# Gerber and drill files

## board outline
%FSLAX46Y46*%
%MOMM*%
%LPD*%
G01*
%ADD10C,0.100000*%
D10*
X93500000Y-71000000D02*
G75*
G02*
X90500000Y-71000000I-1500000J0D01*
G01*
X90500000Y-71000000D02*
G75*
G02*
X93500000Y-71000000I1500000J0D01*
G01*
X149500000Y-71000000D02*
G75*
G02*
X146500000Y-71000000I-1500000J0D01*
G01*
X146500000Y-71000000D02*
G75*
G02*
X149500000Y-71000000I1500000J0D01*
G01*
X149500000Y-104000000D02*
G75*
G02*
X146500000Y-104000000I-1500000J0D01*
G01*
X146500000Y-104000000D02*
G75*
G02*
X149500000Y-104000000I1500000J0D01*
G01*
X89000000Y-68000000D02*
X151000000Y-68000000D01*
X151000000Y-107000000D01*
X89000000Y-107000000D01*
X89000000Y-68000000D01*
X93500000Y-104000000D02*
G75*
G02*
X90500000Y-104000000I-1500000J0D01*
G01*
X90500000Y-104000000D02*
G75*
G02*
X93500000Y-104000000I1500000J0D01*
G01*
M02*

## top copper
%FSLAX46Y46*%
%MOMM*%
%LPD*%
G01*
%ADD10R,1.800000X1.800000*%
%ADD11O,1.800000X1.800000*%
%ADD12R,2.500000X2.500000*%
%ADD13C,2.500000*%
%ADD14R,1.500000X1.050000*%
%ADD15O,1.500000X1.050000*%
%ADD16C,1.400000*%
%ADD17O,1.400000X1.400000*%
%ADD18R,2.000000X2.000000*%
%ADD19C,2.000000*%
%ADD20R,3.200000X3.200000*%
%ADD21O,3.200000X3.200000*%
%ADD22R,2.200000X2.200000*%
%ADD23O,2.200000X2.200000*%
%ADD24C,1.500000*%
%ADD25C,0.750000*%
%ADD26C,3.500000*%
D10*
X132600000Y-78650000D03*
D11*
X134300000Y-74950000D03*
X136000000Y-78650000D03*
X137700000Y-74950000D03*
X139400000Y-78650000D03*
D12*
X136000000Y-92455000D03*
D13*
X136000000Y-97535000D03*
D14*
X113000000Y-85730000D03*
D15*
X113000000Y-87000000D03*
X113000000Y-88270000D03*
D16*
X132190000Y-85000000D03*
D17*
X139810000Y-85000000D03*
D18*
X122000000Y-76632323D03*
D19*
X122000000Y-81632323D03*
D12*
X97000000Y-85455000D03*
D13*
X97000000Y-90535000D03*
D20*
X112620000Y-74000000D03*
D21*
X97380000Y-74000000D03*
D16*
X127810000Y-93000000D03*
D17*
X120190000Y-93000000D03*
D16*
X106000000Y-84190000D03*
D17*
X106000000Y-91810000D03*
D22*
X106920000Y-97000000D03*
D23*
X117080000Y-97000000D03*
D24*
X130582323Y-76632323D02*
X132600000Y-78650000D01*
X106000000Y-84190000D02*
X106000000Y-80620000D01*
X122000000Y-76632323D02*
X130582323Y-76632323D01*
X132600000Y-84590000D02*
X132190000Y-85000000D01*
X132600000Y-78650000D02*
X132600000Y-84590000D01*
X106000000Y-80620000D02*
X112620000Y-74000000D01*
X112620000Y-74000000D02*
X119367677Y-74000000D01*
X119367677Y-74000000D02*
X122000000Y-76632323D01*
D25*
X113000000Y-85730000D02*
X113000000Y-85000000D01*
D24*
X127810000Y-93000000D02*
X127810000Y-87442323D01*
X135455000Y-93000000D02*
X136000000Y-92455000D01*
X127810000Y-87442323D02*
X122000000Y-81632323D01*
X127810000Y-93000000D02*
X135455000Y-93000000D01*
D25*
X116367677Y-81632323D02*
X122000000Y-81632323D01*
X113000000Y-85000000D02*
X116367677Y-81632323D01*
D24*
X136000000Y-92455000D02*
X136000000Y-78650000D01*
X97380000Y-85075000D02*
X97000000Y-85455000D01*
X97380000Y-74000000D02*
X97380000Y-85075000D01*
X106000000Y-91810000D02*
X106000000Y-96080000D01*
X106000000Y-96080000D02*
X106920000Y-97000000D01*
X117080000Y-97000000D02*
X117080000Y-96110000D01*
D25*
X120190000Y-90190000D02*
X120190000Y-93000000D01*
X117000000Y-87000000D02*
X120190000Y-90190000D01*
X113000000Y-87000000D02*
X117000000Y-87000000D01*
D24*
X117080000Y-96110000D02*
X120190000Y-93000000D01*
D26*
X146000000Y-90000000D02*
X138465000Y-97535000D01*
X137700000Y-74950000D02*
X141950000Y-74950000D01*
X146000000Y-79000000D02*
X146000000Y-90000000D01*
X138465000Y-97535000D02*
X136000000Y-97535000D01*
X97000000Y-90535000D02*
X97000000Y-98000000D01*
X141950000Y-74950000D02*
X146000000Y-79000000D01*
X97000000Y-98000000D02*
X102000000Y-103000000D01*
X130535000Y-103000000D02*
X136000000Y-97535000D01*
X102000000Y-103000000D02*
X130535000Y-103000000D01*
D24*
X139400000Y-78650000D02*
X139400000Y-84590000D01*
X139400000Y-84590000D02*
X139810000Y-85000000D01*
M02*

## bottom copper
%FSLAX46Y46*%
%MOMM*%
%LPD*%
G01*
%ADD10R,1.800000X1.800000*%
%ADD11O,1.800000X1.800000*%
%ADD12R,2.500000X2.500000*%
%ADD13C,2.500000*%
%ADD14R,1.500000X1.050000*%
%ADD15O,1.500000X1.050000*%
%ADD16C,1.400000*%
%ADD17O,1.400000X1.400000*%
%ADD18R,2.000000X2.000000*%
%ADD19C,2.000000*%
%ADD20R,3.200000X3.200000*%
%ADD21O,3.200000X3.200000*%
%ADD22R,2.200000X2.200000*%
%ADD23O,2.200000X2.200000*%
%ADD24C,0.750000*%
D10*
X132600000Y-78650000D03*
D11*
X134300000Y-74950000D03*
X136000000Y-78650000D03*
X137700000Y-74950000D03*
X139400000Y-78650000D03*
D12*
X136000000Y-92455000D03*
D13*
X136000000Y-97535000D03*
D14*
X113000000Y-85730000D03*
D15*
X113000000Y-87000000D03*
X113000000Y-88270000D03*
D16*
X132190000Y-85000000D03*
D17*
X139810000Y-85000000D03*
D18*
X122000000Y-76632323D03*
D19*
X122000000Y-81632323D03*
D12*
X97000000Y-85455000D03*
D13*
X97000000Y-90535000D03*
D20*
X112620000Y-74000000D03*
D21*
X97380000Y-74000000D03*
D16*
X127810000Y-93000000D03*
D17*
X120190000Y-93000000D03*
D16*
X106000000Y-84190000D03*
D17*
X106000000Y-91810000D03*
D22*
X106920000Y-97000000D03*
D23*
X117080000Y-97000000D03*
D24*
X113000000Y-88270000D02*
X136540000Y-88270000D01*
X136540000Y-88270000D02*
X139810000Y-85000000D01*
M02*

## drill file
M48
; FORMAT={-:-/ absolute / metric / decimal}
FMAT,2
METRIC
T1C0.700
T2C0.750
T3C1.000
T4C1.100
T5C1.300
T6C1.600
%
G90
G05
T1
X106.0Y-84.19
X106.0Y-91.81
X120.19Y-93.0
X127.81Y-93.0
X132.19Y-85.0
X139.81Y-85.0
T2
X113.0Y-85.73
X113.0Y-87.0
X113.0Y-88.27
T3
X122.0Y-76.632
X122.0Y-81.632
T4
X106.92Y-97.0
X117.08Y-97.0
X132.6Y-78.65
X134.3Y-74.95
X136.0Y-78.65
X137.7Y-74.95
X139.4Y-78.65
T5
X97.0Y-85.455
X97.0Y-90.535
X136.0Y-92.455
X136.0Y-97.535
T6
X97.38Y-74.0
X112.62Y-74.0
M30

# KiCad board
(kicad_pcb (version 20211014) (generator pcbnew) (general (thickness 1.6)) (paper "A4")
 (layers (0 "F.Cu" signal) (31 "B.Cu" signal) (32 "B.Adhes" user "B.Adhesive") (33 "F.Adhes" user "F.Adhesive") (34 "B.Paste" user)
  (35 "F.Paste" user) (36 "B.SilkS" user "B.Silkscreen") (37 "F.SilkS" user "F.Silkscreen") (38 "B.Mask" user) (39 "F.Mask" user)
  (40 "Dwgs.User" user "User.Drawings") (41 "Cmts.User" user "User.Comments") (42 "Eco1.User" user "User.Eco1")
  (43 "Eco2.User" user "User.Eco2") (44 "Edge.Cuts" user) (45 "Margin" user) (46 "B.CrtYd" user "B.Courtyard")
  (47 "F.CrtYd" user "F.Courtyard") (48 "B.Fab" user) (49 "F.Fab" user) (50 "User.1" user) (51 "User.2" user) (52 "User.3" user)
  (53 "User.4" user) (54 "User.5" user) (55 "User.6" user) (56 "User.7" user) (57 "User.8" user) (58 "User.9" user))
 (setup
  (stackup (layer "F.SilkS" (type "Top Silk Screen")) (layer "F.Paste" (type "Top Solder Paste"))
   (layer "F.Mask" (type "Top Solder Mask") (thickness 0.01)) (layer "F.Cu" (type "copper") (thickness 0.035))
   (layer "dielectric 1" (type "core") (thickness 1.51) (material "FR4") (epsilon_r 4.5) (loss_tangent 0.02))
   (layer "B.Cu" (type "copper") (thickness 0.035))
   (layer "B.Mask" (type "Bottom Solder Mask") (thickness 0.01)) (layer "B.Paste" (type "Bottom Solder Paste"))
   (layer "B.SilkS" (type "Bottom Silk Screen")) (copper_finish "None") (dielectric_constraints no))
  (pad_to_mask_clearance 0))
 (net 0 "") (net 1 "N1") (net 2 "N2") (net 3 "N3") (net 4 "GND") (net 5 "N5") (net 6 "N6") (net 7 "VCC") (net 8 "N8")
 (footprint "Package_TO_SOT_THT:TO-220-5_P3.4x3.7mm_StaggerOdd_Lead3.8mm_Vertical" (layer "F.Cu") (at 132.6 78.65)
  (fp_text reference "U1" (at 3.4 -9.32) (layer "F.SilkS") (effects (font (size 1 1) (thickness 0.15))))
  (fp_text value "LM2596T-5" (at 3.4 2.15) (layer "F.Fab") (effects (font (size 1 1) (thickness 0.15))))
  (pad "1" thru_hole rect (at 0 0) (size 1.8 1.8) (drill 1.1) (layers *.Cu *.Mask) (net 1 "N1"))
  (pad "2" thru_hole oval (at 1.7 -3.7) (size 1.8 1.8) (drill 1.1) (layers *.Cu *.Mask) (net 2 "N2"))
  (pad "3" thru_hole oval (at 3.4 0) (size 1.8 1.8) (drill 1.1) (layers *.Cu *.Mask) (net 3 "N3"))
  (pad "4" thru_hole oval (at 5.1 -3.7) (size 1.8 1.8) (drill 1.1) (layers *.Cu *.Mask) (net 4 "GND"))
  (pad "5" thru_hole oval (at 6.8 0) (size 1.8 1.8) (drill 1.1) (layers *.Cu *.Mask) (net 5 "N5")))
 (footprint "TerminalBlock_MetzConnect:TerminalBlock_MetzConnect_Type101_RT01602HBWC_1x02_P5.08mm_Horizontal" (layer "F.Cu")
  (at 136 92.455 -90)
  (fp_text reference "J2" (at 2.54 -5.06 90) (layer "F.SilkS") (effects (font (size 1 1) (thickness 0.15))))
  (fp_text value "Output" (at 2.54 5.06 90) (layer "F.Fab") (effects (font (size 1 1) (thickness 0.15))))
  (pad "1" thru_hole rect (at 0 0 270) (size 2.5 2.5) (drill 1.3) (layers *.Cu *.Mask) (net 3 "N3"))
  (pad "2" thru_hole circle (at 5.08 0 270) (size 2.5 2.5) (drill 1.3) (layers *.Cu *.Mask) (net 4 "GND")))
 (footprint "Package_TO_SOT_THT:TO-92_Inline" (layer "F.Cu") (at 113 85.73 -90)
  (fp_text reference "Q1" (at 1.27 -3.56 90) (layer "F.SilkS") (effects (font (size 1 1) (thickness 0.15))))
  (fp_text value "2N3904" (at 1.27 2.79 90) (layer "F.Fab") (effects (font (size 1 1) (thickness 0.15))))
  (pad "1" thru_hole rect (at 0 0 270) (size 1.05 1.5) (drill 0.75) (layers *.Cu *.Mask) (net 3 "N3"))
  (pad "2" thru_hole oval (at 1.27 0 270) (size 1.05 1.5) (drill 0.75) (layers *.Cu *.Mask) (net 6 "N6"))
  (pad "3" thru_hole oval (at 2.54 0 270) (size 1.05 1.5) (drill 0.75) (layers *.Cu *.Mask) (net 5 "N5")))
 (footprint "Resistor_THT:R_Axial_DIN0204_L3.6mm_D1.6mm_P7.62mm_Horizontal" (layer "F.Cu") (at 132.19 85)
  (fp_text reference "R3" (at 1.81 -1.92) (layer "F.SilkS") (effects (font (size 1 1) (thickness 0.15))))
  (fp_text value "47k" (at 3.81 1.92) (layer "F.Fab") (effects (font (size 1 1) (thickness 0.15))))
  (pad "1" thru_hole circle (at 0 0) (size 1.4 1.4) (drill 0.7) (layers *.Cu *.Mask) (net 1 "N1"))
  (pad "2" thru_hole oval (at 7.62 0) (size 1.4 1.4) (drill 0.7) (layers *.Cu *.Mask) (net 5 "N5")))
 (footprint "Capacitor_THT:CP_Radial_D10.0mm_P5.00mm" (layer "F.Cu") (at 122 76.632323 -90)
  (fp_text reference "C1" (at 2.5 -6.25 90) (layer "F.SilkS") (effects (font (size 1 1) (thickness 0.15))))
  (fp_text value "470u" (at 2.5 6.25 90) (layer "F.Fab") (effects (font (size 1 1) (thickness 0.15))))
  (pad "1" thru_hole rect (at 0 0 270) (size 2 2) (drill 1) (layers *.Cu *.Mask) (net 1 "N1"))
  (pad "2" thru_hole circle (at 5 0 270) (size 2 2) (drill 1) (layers *.Cu *.Mask) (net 3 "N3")))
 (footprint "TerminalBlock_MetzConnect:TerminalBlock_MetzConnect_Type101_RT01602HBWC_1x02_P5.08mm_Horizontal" (layer "F.Cu")
  (at 97 85.455 -90)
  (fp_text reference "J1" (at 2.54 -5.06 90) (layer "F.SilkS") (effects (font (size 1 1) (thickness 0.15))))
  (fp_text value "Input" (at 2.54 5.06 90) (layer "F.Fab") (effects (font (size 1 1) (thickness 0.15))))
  (pad "1" thru_hole rect (at 0 0 270) (size 2.5 2.5) (drill 1.3) (layers *.Cu *.Mask) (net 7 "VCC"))
  (pad "2" thru_hole circle (at 5.08 0 270) (size 2.5 2.5) (drill 1.3) (layers *.Cu *.Mask) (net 4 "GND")))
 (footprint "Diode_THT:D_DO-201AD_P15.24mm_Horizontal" (layer "F.Cu") (at 112.62 74 180)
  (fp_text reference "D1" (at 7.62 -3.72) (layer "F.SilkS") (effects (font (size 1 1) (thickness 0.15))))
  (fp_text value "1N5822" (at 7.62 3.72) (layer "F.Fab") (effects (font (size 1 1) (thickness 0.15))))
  (pad "1" thru_hole rect (at 0 0 180) (size 3.2 3.2) (drill 1.6) (layers *.Cu *.Mask) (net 1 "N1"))
  (pad "2" thru_hole oval (at 15.24 0 180) (size 3.2 3.2) (drill 1.6) (layers *.Cu *.Mask) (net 7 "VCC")))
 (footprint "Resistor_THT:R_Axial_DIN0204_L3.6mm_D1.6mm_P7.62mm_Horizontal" (layer "F.Cu") (at 127.81 93 180)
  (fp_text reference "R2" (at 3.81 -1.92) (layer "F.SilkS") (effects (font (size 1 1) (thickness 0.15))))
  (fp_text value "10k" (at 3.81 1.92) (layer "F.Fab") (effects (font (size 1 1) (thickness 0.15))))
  (pad "1" thru_hole circle (at 0 0 180) (size 1.4 1.4) (drill 0.7) (layers *.Cu *.Mask) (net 3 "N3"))
  (pad "2" thru_hole oval (at 7.62 0 180) (size 1.4 1.4) (drill 0.7) (layers *.Cu *.Mask) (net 6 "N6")))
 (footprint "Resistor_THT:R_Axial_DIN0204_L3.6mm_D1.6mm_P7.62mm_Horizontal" (layer "F.Cu") (at 106 84.19 -90)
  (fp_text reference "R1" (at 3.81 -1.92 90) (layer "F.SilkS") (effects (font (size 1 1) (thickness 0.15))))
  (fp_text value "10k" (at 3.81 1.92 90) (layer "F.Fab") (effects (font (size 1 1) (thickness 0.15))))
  (pad "1" thru_hole circle (at 0 0 270) (size 1.4 1.4) (drill 0.7) (layers *.Cu *.Mask) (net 1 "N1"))
  (pad "2" thru_hole oval (at 7.62 0 270) (size 1.4 1.4) (drill 0.7) (layers *.Cu *.Mask) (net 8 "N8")))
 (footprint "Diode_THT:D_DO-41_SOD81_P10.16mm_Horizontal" (layer "F.Cu") (at 106.92 97)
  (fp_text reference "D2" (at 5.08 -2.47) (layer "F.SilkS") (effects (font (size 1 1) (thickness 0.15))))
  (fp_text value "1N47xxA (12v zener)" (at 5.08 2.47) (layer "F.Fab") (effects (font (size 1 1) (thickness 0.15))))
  (pad "1" thru_hole rect (at 0 0) (size 2.2 2.2) (drill 1.1) (layers *.Cu *.Mask) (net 8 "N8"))
  (pad "2" thru_hole oval (at 10.16 0) (size 2.2 2.2) (drill 1.1) (layers *.Cu *.Mask) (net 6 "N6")))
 (gr_circle (center 92 71) (end 93.5 71) (layer "Edge.Cuts") (width 0.1) (fill none))
 (gr_circle (center 148 71) (end 149.5 71) (layer "Edge.Cuts") (width 0.1) (fill none))
 (gr_circle (center 148 104) (end 149.5 104) (layer "Edge.Cuts") (width 0.1) (fill none))
 (gr_rect (start 89 68) (end 151 107) (layer "Edge.Cuts") (width 0.1) (fill none))
 (gr_circle (center 92 104) (end 93.5 104) (layer "Edge.Cuts") (width 0.1) (fill none))
 (segment (start 130.582323 76.632323) (end 132.6 78.65) (width 1.5) (layer "F.Cu") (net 1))
 (segment (start 106 84.19) (end 106 80.62) (width 1.5) (layer "F.Cu") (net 1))
 (segment (start 122 76.632323) (end 130.582323 76.632323) (width 1.5) (layer "F.Cu") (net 1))
 (segment (start 132.6 84.59) (end 132.19 85) (width 1.5) (layer "F.Cu") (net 1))
 (segment (start 132.6 78.65) (end 132.6 84.59) (width 1.5) (layer "F.Cu") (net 1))
 (segment (start 106 80.62) (end 112.62 74) (width 1.5) (layer "F.Cu") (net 1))
 (segment (start 112.62 74) (end 119.367677 74) (width 1.5) (layer "F.Cu") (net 1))
 (segment (start 119.367677 74) (end 122 76.632323) (width 1.5) (layer "F.Cu") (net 1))
 (segment (start 113 85.73) (end 113 85) (width 0.75) (layer "F.Cu") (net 3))
 (segment (start 127.81 93) (end 127.81 87.442323) (width 1.5) (layer "F.Cu") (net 3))
 (segment (start 135.455 93) (end 136 92.455) (width 1.5) (layer "F.Cu") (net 3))
 (segment (start 127.81 87.442323) (end 122 81.632323) (width 1.5) (layer "F.Cu") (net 3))
 (segment (start 127.81 93) (end 135.455 93) (width 1.5) (layer "F.Cu") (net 3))
 (segment (start 116.367677 81.632323) (end 122 81.632323) (width 0.75) (layer "F.Cu") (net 3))
 (segment (start 113 85) (end 116.367677 81.632323) (width 0.75) (layer "F.Cu") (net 3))
 (segment (start 136 92.455) (end 136 78.65) (width 1.5) (layer "F.Cu") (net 3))
 (segment (start 97.38 85.075) (end 97 85.455) (width 1.5) (layer "F.Cu") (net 7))
 (segment (start 97.38 74) (end 97.38 85.075) (width 1.5) (layer "F.Cu") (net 7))
 (segment (start 106 91.81) (end 106 96.08) (width 1.5) (layer "F.Cu") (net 8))
 (segment (start 106 96.08) (end 106.92 97) (width 1.5) (layer "F.Cu") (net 8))
 (segment (start 117.08 97) (end 117.08 96.11) (width 1.5) (layer "F.Cu") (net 6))
 (segment (start 120.19 90.19) (end 120.19 93) (width 0.75) (layer "F.Cu") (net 6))
 (segment (start 117 87) (end 120.19 90.19) (width 0.75) (layer "F.Cu") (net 6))
 (segment (start 113 87) (end 117 87) (width 0.75) (layer "F.Cu") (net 6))
 (segment (start 117.08 96.11) (end 120.19 93) (width 1.5) (layer "F.Cu") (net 6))
 (segment (start 146 90) (end 138.465 97.535) (width 3.5) (layer "F.Cu") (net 4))
 (segment (start 137.7 74.95) (end 141.95 74.95) (width 3.5) (layer "F.Cu") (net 4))
 (segment (start 146 79) (end 146 90) (width 3.5) (layer "F.Cu") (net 4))
 (segment (start 138.465 97.535) (end 136 97.535) (width 3.5) (layer "F.Cu") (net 4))
 (segment (start 97 90.535) (end 97 98) (width 3.5) (layer "F.Cu") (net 4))
 (segment (start 141.95 74.95) (end 146 79) (width 3.5) (layer "F.Cu") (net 4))
 (segment (start 97 98) (end 102 103) (width 3.5) (layer "F.Cu") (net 4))
 (segment (start 130.535 103) (end 136 97.535) (width 3.5) (layer "F.Cu") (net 4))
 (segment (start 102 103) (end 130.535 103) (width 3.5) (layer "F.Cu") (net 4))
 (segment (start 139.4 78.65) (end 139.4 84.59) (width 1.5) (layer "F.Cu") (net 5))
 (segment (start 139.4 84.59) (end 139.81 85) (width 1.5) (layer "F.Cu") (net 5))
 (segment (start 113 88.27) (end 136.54 88.27) (width 0.75) (layer "B.Cu") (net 5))
 (segment (start 136.54 88.27) (end 139.81 85) (width 0.75) (layer "B.Cu") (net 5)))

